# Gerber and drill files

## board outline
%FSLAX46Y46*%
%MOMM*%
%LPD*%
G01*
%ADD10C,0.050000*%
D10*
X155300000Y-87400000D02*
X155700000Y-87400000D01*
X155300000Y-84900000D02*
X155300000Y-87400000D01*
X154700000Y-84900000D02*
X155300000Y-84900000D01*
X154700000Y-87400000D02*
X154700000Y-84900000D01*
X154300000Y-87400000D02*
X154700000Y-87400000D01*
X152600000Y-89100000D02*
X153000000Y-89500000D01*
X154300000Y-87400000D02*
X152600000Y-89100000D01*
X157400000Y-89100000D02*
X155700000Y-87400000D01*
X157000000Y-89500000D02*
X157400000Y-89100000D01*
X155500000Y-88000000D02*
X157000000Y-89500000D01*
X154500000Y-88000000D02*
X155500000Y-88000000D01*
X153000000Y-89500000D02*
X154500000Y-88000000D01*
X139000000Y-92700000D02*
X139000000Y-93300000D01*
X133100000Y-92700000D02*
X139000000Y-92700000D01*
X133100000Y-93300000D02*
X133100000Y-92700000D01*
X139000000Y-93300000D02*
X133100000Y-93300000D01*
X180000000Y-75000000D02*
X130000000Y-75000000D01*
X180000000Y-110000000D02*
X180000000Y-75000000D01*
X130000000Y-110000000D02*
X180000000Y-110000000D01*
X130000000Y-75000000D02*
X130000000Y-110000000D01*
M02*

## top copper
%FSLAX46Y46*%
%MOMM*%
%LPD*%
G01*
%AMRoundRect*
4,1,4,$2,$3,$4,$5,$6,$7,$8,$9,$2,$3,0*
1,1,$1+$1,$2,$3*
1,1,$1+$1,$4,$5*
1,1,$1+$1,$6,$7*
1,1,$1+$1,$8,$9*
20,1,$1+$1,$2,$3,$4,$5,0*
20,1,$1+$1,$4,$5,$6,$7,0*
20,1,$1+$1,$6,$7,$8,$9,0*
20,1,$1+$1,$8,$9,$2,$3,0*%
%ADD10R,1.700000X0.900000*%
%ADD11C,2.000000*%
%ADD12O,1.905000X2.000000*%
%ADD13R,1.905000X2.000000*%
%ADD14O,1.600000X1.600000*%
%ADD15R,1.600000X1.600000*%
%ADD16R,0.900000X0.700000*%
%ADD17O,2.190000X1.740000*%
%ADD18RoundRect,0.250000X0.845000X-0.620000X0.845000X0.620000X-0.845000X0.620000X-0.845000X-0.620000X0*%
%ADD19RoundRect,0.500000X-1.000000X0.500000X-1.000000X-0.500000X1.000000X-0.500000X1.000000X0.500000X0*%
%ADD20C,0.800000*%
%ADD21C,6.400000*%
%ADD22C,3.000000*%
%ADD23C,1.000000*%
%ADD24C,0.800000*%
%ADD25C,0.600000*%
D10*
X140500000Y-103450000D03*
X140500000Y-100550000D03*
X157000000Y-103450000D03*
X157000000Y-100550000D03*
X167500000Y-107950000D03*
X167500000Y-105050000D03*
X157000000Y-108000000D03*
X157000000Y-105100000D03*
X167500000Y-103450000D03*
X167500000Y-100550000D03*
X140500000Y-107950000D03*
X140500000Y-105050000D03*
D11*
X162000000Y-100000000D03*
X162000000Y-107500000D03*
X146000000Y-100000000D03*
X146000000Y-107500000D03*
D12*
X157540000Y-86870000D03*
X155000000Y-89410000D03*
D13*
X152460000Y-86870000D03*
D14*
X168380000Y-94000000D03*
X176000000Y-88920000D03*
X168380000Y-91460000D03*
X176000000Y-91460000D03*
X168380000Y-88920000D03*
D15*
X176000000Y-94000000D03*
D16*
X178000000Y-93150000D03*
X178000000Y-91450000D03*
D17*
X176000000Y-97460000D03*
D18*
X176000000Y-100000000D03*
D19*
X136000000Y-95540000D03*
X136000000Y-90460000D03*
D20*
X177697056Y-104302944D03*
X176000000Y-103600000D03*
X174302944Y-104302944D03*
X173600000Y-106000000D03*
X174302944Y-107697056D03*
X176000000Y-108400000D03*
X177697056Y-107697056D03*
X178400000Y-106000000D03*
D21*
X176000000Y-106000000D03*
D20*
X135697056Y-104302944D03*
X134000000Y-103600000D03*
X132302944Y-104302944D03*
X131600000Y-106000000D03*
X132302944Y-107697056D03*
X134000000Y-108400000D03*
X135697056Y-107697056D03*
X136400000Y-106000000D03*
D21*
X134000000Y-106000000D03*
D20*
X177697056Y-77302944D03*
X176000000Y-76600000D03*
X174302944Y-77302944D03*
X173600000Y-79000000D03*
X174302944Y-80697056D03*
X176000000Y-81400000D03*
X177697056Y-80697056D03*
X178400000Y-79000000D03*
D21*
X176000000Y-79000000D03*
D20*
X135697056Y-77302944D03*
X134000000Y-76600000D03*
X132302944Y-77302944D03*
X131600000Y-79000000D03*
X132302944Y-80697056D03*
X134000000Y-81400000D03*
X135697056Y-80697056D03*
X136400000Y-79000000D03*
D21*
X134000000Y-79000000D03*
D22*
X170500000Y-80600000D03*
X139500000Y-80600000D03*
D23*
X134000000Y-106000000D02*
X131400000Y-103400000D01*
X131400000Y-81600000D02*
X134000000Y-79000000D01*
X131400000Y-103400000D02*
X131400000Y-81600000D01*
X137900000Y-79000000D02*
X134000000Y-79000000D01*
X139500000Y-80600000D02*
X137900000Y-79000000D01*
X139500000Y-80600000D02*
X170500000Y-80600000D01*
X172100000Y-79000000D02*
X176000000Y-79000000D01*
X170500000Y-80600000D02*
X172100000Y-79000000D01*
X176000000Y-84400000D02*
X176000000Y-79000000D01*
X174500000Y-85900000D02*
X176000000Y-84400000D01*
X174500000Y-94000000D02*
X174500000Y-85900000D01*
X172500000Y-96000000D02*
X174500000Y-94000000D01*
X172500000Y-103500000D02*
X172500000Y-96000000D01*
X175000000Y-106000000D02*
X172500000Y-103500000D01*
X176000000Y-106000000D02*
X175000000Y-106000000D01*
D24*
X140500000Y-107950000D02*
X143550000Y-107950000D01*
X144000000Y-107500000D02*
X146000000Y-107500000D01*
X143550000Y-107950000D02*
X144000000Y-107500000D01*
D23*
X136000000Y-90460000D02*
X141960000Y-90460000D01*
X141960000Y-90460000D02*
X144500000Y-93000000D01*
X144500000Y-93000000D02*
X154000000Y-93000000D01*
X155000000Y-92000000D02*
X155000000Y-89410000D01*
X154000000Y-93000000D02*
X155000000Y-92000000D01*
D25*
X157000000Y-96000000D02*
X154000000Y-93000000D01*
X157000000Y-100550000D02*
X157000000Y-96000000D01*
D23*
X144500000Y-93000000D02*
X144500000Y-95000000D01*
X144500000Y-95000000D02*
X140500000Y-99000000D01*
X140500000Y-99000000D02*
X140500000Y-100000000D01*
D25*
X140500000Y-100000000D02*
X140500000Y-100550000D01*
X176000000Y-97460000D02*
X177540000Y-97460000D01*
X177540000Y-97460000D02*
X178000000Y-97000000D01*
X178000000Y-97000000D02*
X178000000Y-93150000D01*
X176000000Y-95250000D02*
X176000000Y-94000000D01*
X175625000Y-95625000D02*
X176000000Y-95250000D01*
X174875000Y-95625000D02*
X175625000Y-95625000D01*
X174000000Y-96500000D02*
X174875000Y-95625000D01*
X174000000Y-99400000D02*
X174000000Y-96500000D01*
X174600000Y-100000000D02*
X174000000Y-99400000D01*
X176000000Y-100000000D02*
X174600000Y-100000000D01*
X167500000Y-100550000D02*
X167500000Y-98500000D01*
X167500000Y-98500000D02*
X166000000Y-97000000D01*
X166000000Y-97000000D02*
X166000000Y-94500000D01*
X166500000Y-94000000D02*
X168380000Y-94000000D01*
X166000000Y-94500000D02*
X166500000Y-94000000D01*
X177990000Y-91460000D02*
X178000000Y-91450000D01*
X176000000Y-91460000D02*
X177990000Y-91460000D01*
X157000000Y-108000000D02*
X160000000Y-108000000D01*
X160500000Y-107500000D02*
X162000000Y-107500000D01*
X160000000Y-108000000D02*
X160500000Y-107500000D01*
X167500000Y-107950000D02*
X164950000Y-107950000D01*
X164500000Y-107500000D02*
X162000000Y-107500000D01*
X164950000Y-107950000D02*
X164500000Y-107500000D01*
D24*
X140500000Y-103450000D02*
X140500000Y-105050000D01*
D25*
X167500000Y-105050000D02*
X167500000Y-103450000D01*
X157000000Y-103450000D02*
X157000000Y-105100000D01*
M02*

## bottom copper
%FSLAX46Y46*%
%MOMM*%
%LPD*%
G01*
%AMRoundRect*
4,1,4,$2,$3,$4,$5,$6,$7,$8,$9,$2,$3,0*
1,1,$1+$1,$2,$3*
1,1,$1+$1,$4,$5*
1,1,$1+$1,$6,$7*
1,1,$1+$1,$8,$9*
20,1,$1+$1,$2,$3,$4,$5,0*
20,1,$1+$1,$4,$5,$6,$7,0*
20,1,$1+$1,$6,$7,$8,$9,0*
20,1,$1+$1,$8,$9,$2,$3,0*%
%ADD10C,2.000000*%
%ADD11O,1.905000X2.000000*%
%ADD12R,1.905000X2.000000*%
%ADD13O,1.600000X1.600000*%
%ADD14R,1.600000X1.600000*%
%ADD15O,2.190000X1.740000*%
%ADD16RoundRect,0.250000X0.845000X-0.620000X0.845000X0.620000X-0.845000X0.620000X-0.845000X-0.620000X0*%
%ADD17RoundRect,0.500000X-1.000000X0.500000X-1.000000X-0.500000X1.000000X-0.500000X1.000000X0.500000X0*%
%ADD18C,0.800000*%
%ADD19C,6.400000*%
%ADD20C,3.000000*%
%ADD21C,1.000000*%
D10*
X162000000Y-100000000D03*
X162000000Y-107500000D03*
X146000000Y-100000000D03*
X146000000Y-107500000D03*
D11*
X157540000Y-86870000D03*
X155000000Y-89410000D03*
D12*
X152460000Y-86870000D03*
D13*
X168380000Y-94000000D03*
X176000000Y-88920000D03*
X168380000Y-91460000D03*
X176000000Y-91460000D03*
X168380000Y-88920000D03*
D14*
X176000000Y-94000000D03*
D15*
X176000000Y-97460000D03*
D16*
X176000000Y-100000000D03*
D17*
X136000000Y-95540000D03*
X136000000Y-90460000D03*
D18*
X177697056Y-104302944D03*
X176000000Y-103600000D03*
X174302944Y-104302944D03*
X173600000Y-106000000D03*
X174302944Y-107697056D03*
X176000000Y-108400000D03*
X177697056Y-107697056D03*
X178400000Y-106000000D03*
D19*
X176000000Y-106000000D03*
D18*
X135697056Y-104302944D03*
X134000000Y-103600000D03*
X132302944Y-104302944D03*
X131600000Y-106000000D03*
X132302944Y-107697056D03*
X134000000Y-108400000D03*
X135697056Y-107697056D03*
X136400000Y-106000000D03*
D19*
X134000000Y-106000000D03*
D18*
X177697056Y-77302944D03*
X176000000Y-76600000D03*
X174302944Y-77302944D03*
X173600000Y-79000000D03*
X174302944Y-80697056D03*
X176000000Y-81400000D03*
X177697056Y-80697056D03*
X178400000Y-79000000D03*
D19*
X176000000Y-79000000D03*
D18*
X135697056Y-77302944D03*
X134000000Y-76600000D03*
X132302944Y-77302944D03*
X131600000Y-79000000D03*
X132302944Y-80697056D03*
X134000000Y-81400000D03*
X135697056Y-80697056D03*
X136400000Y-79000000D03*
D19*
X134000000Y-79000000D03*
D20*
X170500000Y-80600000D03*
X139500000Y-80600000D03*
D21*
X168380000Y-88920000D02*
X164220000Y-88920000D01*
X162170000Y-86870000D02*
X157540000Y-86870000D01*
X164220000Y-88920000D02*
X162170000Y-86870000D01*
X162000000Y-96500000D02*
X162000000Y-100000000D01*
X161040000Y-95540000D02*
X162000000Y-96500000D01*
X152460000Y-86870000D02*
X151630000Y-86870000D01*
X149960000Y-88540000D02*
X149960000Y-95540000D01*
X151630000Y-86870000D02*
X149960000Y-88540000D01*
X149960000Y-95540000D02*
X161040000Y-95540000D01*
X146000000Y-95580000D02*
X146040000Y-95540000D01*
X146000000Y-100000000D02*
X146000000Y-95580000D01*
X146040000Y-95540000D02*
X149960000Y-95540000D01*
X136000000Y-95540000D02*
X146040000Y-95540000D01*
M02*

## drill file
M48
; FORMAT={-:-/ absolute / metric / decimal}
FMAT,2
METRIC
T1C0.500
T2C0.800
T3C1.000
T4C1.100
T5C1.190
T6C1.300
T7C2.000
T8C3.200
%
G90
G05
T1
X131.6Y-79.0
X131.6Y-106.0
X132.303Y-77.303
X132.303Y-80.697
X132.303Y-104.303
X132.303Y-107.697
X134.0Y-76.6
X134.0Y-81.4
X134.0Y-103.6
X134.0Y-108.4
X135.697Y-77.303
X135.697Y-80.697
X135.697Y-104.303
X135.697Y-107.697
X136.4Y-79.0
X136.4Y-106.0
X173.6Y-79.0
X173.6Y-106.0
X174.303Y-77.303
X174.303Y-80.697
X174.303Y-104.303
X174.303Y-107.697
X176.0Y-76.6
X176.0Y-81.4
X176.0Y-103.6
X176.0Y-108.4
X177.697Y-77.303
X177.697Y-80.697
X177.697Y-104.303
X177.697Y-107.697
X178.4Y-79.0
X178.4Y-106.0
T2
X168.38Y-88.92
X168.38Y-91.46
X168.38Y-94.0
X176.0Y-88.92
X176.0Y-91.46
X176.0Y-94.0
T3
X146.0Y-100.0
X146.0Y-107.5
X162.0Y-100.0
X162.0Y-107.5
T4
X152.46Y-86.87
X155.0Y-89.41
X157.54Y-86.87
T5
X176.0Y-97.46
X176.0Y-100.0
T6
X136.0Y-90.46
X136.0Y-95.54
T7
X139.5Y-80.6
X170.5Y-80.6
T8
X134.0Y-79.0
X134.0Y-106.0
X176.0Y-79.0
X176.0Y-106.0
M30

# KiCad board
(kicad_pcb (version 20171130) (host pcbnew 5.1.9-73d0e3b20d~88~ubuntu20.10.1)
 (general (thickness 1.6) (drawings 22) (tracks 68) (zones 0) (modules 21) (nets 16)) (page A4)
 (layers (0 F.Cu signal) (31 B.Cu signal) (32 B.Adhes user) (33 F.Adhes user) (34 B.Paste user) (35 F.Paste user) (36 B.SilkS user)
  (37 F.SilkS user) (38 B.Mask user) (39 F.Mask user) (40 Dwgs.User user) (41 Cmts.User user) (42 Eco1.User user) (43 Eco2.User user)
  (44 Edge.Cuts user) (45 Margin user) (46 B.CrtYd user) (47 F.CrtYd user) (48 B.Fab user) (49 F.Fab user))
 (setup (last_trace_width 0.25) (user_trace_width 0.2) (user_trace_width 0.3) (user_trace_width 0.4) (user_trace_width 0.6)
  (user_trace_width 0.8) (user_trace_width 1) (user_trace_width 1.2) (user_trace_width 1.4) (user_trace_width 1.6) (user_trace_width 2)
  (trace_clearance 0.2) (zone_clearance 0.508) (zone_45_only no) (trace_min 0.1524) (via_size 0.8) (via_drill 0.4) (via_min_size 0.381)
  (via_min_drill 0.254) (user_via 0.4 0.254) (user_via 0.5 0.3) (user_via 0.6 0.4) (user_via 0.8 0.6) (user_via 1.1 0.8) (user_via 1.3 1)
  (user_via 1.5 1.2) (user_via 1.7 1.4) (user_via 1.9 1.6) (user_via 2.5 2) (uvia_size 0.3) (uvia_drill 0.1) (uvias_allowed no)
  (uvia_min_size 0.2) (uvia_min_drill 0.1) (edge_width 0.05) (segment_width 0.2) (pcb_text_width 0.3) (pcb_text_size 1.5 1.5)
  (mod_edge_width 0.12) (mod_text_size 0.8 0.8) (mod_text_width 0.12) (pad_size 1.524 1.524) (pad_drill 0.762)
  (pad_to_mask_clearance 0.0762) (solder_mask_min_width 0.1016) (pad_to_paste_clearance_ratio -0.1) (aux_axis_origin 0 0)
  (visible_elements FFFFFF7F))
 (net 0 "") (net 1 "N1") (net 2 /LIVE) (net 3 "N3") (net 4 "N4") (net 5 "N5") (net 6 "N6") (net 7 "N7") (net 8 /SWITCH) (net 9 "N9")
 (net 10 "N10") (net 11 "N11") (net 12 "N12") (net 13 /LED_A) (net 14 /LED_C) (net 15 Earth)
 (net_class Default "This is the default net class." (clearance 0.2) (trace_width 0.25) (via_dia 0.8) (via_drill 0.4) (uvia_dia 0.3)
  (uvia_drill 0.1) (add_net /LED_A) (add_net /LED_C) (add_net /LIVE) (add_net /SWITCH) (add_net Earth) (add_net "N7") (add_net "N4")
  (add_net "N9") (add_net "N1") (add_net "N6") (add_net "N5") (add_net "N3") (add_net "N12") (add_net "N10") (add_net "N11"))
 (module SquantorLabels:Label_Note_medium (layer F.Cu) (at 156.5 94.2)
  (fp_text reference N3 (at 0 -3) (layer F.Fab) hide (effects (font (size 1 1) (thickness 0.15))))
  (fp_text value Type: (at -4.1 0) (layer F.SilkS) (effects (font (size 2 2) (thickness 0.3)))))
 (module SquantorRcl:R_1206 (layer F.Cu) (at 140.5 102 270)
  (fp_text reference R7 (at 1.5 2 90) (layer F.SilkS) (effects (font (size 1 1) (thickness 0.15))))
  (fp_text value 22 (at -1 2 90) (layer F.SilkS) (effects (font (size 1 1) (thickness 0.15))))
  (pad 2 smd rect (at 1.45 0 270) (size 0.9 1.7) (layers F.Cu F.Paste F.Mask) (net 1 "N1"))
  (pad 1 smd rect (at -1.45 0 270) (size 0.9 1.7) (layers F.Cu F.Paste F.Mask) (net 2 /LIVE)))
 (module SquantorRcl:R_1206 (layer F.Cu) (at 157 102 270)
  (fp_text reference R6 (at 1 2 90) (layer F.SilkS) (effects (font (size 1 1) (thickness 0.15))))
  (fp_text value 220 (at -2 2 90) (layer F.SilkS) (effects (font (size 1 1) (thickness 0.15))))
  (pad 2 smd rect (at 1.45 0 270) (size 0.9 1.7) (layers F.Cu F.Paste F.Mask) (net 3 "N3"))
  (pad 1 smd rect (at -1.45 0 270) (size 0.9 1.7) (layers F.Cu F.Paste F.Mask) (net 2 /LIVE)))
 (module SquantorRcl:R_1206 (layer F.Cu) (at 167.5 106.5 270)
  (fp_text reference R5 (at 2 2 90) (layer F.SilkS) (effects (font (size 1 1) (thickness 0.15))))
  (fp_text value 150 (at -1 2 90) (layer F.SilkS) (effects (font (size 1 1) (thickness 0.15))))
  (pad 2 smd rect (at 1.45 0 270) (size 0.9 1.7) (layers F.Cu F.Paste F.Mask) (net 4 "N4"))
  (pad 1 smd rect (at -1.45 0 270) (size 0.9 1.7) (layers F.Cu F.Paste F.Mask) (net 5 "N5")))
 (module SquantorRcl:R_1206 (layer F.Cu) (at 157 106.55 270)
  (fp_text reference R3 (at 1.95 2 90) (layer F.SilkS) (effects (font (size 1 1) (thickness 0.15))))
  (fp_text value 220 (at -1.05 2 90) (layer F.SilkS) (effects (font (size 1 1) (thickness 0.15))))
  (pad 2 smd rect (at 1.45 0 270) (size 0.9 1.7) (layers F.Cu F.Paste F.Mask) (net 4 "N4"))
  (pad 1 smd rect (at -1.45 0 270) (size 0.9 1.7) (layers F.Cu F.Paste F.Mask) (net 3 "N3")))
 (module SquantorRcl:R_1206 (layer F.Cu) (at 167.5 102 270)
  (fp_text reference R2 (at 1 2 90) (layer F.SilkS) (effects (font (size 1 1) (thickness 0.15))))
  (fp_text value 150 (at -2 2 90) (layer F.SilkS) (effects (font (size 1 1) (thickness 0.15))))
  (pad 2 smd rect (at 1.45 0 270) (size 0.9 1.7) (layers F.Cu F.Paste F.Mask) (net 5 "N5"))
  (pad 1 smd rect (at -1.45 0 270) (size 0.9 1.7) (layers F.Cu F.Paste F.Mask) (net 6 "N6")))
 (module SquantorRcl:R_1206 (layer F.Cu) (at 140.5 106.5 270)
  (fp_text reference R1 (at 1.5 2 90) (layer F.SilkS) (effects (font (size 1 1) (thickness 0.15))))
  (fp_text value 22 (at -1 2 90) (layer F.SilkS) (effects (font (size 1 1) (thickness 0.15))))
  (pad 2 smd rect (at 1.45 0 270) (size 0.9 1.7) (layers F.Cu F.Paste F.Mask) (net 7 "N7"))
  (pad 1 smd rect (at -1.45 0 270) (size 0.9 1.7) (layers F.Cu F.Paste F.Mask) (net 1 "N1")))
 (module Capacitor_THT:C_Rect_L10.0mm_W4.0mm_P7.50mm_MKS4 (layer F.Cu) (at 162 107.5 90)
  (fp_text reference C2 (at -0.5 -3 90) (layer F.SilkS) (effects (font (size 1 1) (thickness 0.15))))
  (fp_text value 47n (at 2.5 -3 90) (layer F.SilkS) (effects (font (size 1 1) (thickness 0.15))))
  (pad 2 thru_hole circle (at 7.5 0 90) (size 2 2) (drill 1) (layers *.Cu *.Mask) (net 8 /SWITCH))
  (pad 1 thru_hole circle (at 0 0 90) (size 2 2) (drill 1) (layers *.Cu *.Mask) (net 4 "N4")))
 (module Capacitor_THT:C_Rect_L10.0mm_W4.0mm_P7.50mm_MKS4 (layer F.Cu) (at 146 107.5 90)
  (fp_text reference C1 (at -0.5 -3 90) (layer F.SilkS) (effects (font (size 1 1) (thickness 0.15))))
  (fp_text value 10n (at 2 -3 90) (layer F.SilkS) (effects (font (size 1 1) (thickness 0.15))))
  (pad 2 thru_hole circle (at 7.5 0 90) (size 2 2) (drill 1) (layers *.Cu *.Mask) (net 8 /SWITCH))
  (pad 1 thru_hole circle (at 0 0 90) (size 2 2) (drill 1) (layers *.Cu *.Mask) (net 7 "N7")))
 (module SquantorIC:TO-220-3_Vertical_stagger (layer F.Cu) (at 155 85.6)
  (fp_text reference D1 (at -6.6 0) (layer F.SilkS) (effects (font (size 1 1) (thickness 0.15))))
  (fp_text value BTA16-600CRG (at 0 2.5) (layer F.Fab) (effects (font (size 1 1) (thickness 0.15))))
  (pad 3 thru_hole oval (at 2.54 1.27) (size 1.905 2) (drill 1.1) (layers *.Cu *.Mask) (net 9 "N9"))
  (pad 2 thru_hole oval (at 0 3.81) (size 1.905 2) (drill 1.1) (layers *.Cu *.Mask) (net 2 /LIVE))
  (pad 1 thru_hole rect (at -2.54 1.27) (size 1.905 2) (drill 1.1) (layers *.Cu *.Mask) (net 8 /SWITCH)))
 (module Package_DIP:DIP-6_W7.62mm (layer F.Cu) (at 176 94 180)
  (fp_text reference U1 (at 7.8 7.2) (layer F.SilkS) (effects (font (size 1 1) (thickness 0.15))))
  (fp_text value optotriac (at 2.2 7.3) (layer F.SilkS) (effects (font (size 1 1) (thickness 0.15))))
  (pad 6 thru_hole oval (at 7.62 0 180) (size 1.6 1.6) (drill 0.8) (layers *.Cu *.Mask) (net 6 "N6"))
  (pad 3 thru_hole oval (at 0 5.08 180) (size 1.6 1.6) (drill 0.8) (layers *.Cu *.Mask) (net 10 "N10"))
  (pad 5 thru_hole oval (at 7.62 2.54 180) (size 1.6 1.6) (drill 0.8) (layers *.Cu *.Mask) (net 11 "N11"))
  (pad 2 thru_hole oval (at 0 2.54 180) (size 1.6 1.6) (drill 0.8) (layers *.Cu *.Mask) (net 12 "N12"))
  (pad 4 thru_hole oval (at 7.62 5.08 180) (size 1.6 1.6) (drill 0.8) (layers *.Cu *.Mask) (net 9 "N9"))
  (pad 1 thru_hole rect (at 0 0 180) (size 1.6 1.6) (drill 0.8) (layers *.Cu *.Mask) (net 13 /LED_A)))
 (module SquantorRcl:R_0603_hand (layer F.Cu) (at 178 92.3 270)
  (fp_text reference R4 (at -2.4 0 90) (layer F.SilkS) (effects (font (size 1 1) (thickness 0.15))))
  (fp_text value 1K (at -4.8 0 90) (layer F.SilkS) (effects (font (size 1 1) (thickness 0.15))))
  (pad 2 smd rect (at 0.85 0 270) (size 0.7 0.9) (layers F.Cu F.Paste F.Mask) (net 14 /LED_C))
  (pad 1 smd rect (at -0.85 0 270) (size 0.7 0.9) (layers F.Cu F.Paste F.Mask) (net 12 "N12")))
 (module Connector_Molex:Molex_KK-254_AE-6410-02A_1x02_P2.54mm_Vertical (layer F.Cu) (at 176 100 90)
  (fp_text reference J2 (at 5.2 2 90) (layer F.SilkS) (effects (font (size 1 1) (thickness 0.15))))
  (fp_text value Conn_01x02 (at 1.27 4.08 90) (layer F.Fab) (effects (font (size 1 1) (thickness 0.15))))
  (pad 2 thru_hole oval (at 2.54 0 90) (size 1.74 2.19) (drill 1.19) (layers *.Cu *.Mask) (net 14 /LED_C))
  (pad 1 thru_hole roundrect (at 0 0 90) (size 1.74 2.19) (drill 1.19) (layers *.Cu *.Mask) (roundrect_rratio 0.143678) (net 13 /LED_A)))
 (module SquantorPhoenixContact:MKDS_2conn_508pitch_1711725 (layer F.Cu) (at 136 93 270)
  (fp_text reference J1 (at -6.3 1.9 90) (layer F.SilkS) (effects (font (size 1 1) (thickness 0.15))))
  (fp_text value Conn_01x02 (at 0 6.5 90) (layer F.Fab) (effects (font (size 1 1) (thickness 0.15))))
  (pad 2 thru_hole roundrect (at 2.54 0 270) (size 2 3) (drill 1.3) (layers *.Cu *.Mask) (roundrect_rratio 0.25) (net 8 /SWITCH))
  (pad 1 thru_hole roundrect (at -2.54 0 270) (size 2 3) (drill 1.3) (layers *.Cu *.Mask) (roundrect_rratio 0.25) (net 2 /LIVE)))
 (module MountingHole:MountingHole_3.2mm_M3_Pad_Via (layer F.Cu) (at 176 106)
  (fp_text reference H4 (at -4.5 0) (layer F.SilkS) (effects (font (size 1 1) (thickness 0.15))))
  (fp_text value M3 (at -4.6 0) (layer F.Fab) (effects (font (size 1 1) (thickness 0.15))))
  (pad 1 thru_hole circle (at 1.697056 -1.697056) (size 0.8 0.8) (drill 0.5) (layers *.Cu *.Mask) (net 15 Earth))
  (pad 1 thru_hole circle (at 0 -2.4) (size 0.8 0.8) (drill 0.5) (layers *.Cu *.Mask) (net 15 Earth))
  (pad 1 thru_hole circle (at -1.697056 -1.697056) (size 0.8 0.8) (drill 0.5) (layers *.Cu *.Mask) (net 15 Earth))
  (pad 1 thru_hole circle (at -2.4 0) (size 0.8 0.8) (drill 0.5) (layers *.Cu *.Mask) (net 15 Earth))
  (pad 1 thru_hole circle (at -1.697056 1.697056) (size 0.8 0.8) (drill 0.5) (layers *.Cu *.Mask) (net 15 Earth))
  (pad 1 thru_hole circle (at 0 2.4) (size 0.8 0.8) (drill 0.5) (layers *.Cu *.Mask) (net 15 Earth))
  (pad 1 thru_hole circle (at 1.697056 1.697056) (size 0.8 0.8) (drill 0.5) (layers *.Cu *.Mask) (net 15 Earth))
  (pad 1 thru_hole circle (at 2.4 0) (size 0.8 0.8) (drill 0.5) (layers *.Cu *.Mask) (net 15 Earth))
  (pad 1 thru_hole circle (at 0 0) (size 6.4 6.4) (drill 3.2) (layers *.Cu *.Mask) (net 15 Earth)))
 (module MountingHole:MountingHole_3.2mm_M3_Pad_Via (layer F.Cu) (at 134 106)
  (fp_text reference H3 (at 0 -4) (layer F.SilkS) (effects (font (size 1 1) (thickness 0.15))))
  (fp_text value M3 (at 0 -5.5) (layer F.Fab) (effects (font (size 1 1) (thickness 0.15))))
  (pad 1 thru_hole circle (at 1.697056 -1.697056) (size 0.8 0.8) (drill 0.5) (layers *.Cu *.Mask) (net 15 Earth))
  (pad 1 thru_hole circle (at 0 -2.4) (size 0.8 0.8) (drill 0.5) (layers *.Cu *.Mask) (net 15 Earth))
  (pad 1 thru_hole circle (at -1.697056 -1.697056) (size 0.8 0.8) (drill 0.5) (layers *.Cu *.Mask) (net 15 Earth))
  (pad 1 thru_hole circle (at -2.4 0) (size 0.8 0.8) (drill 0.5) (layers *.Cu *.Mask) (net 15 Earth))
  (pad 1 thru_hole circle (at -1.697056 1.697056) (size 0.8 0.8) (drill 0.5) (layers *.Cu *.Mask) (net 15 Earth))
  (pad 1 thru_hole circle (at 0 2.4) (size 0.8 0.8) (drill 0.5) (layers *.Cu *.Mask) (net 15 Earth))
  (pad 1 thru_hole circle (at 1.697056 1.697056) (size 0.8 0.8) (drill 0.5) (layers *.Cu *.Mask) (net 15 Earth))
  (pad 1 thru_hole circle (at 2.4 0) (size 0.8 0.8) (drill 0.5) (layers *.Cu *.Mask) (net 15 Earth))
  (pad 1 thru_hole circle (at 0 0) (size 6.4 6.4) (drill 3.2) (layers *.Cu *.Mask) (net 15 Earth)))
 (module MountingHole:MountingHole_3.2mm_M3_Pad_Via (layer F.Cu) (at 176 79)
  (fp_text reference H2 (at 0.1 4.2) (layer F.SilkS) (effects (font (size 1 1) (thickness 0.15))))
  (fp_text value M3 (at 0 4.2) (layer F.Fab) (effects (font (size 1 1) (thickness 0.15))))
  (pad 1 thru_hole circle (at 1.697056 -1.697056) (size 0.8 0.8) (drill 0.5) (layers *.Cu *.Mask) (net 15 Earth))
  (pad 1 thru_hole circle (at 0 -2.4) (size 0.8 0.8) (drill 0.5) (layers *.Cu *.Mask) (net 15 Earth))
  (pad 1 thru_hole circle (at -1.697056 -1.697056) (size 0.8 0.8) (drill 0.5) (layers *.Cu *.Mask) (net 15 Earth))
  (pad 1 thru_hole circle (at -2.4 0) (size 0.8 0.8) (drill 0.5) (layers *.Cu *.Mask) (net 15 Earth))
  (pad 1 thru_hole circle (at -1.697056 1.697056) (size 0.8 0.8) (drill 0.5) (layers *.Cu *.Mask) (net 15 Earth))
  (pad 1 thru_hole circle (at 0 2.4) (size 0.8 0.8) (drill 0.5) (layers *.Cu *.Mask) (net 15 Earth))
  (pad 1 thru_hole circle (at 1.697056 1.697056) (size 0.8 0.8) (drill 0.5) (layers *.Cu *.Mask) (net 15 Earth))
  (pad 1 thru_hole circle (at 2.4 0) (size 0.8 0.8) (drill 0.5) (layers *.Cu *.Mask) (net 15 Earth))
  (pad 1 thru_hole circle (at 0 0) (size 6.4 6.4) (drill 3.2) (layers *.Cu *.Mask) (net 15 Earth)))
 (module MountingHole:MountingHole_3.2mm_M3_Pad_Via (layer F.Cu) (at 134 79)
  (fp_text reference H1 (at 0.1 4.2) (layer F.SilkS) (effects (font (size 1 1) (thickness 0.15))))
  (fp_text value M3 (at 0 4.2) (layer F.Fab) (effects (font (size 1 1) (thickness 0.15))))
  (pad 1 thru_hole circle (at 1.697056 -1.697056) (size 0.8 0.8) (drill 0.5) (layers *.Cu *.Mask) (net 15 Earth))
  (pad 1 thru_hole circle (at 0 -2.4) (size 0.8 0.8) (drill 0.5) (layers *.Cu *.Mask) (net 15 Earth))
  (pad 1 thru_hole circle (at -1.697056 -1.697056) (size 0.8 0.8) (drill 0.5) (layers *.Cu *.Mask) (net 15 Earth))
  (pad 1 thru_hole circle (at -2.4 0) (size 0.8 0.8) (drill 0.5) (layers *.Cu *.Mask) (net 15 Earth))
  (pad 1 thru_hole circle (at -1.697056 1.697056) (size 0.8 0.8) (drill 0.5) (layers *.Cu *.Mask) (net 15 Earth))
  (pad 1 thru_hole circle (at 0 2.4) (size 0.8 0.8) (drill 0.5) (layers *.Cu *.Mask) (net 15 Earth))
  (pad 1 thru_hole circle (at 1.697056 1.697056) (size 0.8 0.8) (drill 0.5) (layers *.Cu *.Mask) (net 15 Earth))
  (pad 1 thru_hole circle (at 2.4 0) (size 0.8 0.8) (drill 0.5) (layers *.Cu *.Mask) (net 15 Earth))
  (pad 1 thru_hole circle (at 0 0) (size 6.4 6.4) (drill 3.2) (layers *.Cu *.Mask) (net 15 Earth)))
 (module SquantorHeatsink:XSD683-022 (layer F.Cu) (at 155 80.6)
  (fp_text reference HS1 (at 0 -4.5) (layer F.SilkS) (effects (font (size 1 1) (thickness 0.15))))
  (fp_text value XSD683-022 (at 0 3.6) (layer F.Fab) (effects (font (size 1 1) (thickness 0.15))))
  (pad 2 thru_hole circle (at 15.5 0) (size 3 3) (drill 2) (layers *.Cu *.Mask) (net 15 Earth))
  (pad 1 thru_hole circle (at -15.5 0) (size 3 3) (drill 2) (layers *.Cu *.Mask) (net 15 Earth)))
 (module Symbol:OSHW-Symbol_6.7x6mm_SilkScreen (layer B.Cu) (at 155.2 80.2 180)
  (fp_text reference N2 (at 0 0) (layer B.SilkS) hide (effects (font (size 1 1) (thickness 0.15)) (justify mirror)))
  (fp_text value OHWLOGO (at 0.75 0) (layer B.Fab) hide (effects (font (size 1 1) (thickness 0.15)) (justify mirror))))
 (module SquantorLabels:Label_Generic (layer B.Cu) (at 155.8 84.1 180)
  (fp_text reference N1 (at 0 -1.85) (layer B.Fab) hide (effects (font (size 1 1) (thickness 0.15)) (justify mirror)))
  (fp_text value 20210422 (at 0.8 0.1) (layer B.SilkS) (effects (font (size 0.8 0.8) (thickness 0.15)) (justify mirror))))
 (gr_line (start 155.3 87.4) (end 155.7 87.4) (layer Edge.Cuts) (width 0.05))
 (gr_line (start 155.3 84.9) (end 155.3 87.4) (layer Edge.Cuts) (width 0.05))
 (gr_line (start 154.7 84.9) (end 155.3 84.9) (layer Edge.Cuts) (width 0.05))
 (gr_line (start 154.7 87.4) (end 154.7 84.9) (layer Edge.Cuts) (width 0.05))
 (gr_line (start 154.3 87.4) (end 154.7 87.4) (layer Edge.Cuts) (width 0.05))
 (gr_line (start 152.6 89.1) (end 153 89.5) (layer Edge.Cuts) (width 0.05))
 (gr_line (start 154.3 87.4) (end 152.6 89.1) (layer Edge.Cuts) (width 0.05))
 (gr_line (start 157.4 89.1) (end 155.7 87.4) (layer Edge.Cuts) (width 0.05))
 (gr_line (start 157 89.5) (end 157.4 89.1) (layer Edge.Cuts) (width 0.05))
 (gr_line (start 155.5 88) (end 157 89.5) (layer Edge.Cuts) (width 0.05))
 (gr_line (start 154.5 88) (end 155.5 88) (layer Edge.Cuts) (width 0.05))
 (gr_line (start 153 89.5) (end 154.5 88) (layer Edge.Cuts) (width 0.05))
 (gr_line (start 139 92.7) (end 139 93.3) (layer Edge.Cuts) (width 0.05))
 (gr_line (start 133.1 92.7) (end 139 92.7) (layer Edge.Cuts) (width 0.05))
 (gr_line (start 133.1 93.3) (end 133.1 92.7) (layer Edge.Cuts) (width 0.05))
 (gr_line (start 139 93.3) (end 133.1 93.3) (layer Edge.Cuts) (width 0.05))
 (gr_line (start 180 75) (end 130 75) (layer Edge.Cuts) (width 0.05))
 (gr_line (start 180 110) (end 180 75) (layer Edge.Cuts) (width 0.05))
 (gr_line (start 130 110) (end 180 110) (layer Edge.Cuts) (width 0.05))
 (gr_line (start 130 75) (end 130 110) (layer Edge.Cuts) (width 0.05))
 (segment (start 168.38 88.92) (end 164.22 88.92) (width 1) (layer B.Cu) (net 9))
 (segment (start 162.17 86.87) (end 157.54 86.87) (width 1) (layer B.Cu) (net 9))
 (segment (start 164.22 88.92) (end 162.17 86.87) (width 1) (layer B.Cu) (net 9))
 (segment (start 134 106) (end 131.4 103.4) (width 1) (layer F.Cu) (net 15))
 (segment (start 131.4 81.6) (end 134 79) (width 1) (layer F.Cu) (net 15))
 (segment (start 131.4 103.4) (end 131.4 81.6) (width 1) (layer F.Cu) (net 15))
 (segment (start 137.9 79) (end 134 79) (width 1) (layer F.Cu) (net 15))
 (segment (start 139.5 80.6) (end 137.9 79) (width 1) (layer F.Cu) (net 15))
 (segment (start 139.5 80.6) (end 170.5 80.6) (width 1) (layer F.Cu) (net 15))
 (segment (start 172.1 79) (end 176 79) (width 1) (layer F.Cu) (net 15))
 (segment (start 170.5 80.6) (end 172.1 79) (width 1) (layer F.Cu) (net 15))
 (segment (start 176 84.4) (end 176 79) (width 1) (layer F.Cu) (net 15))
 (segment (start 174.5 85.9) (end 176 84.4) (width 1) (layer F.Cu) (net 15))
 (segment (start 174.5 94) (end 174.5 85.9) (width 1) (layer F.Cu) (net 15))
 (segment (start 172.5 96) (end 174.5 94) (width 1) (layer F.Cu) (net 15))
 (segment (start 172.5 103.5) (end 172.5 96) (width 1) (layer F.Cu) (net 15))
 (segment (start 175 106) (end 172.5 103.5) (width 1) (layer F.Cu) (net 15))
 (segment (start 176 106) (end 175 106) (width 1) (layer F.Cu) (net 15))
 (segment (start 140.5 107.95) (end 143.55 107.95) (width 0.8) (layer F.Cu) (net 7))
 (segment (start 144 107.5) (end 146 107.5) (width 0.8) (layer F.Cu) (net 7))
 (segment (start 143.55 107.95) (end 144 107.5) (width 0.8) (layer F.Cu) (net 7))
 (segment (start 136 90.46) (end 141.96 90.46) (width 1) (layer F.Cu) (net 2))
 (segment (start 141.96 90.46) (end 144.5 93) (width 1) (layer F.Cu) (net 2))
 (segment (start 144.5 93) (end 154 93) (width 1) (layer F.Cu) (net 2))
 (segment (start 155 92) (end 155 89.41) (width 1) (layer F.Cu) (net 2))
 (segment (start 154 93) (end 155 92) (width 1) (layer F.Cu) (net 2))
 (segment (start 157 96) (end 154 93) (width 0.6) (layer F.Cu) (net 2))
 (segment (start 157 100.55) (end 157 96) (width 0.6) (layer F.Cu) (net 2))
 (segment (start 144.5 93) (end 144.5 95) (width 1) (layer F.Cu) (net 2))
 (segment (start 144.5 95) (end 140.5 99) (width 1) (layer F.Cu) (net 2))
 (segment (start 140.5 99) (end 140.5 100) (width 1) (layer F.Cu) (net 2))
 (segment (start 140.5 100) (end 140.5 100.55) (width 0.6) (layer F.Cu) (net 2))
 (segment (start 162 96.5) (end 162 100) (width 1) (layer B.Cu) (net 8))
 (segment (start 161.04 95.54) (end 162 96.5) (width 1) (layer B.Cu) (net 8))
 (segment (start 152.46 86.87) (end 151.63 86.87) (width 1) (layer B.Cu) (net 8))
 (segment (start 149.96 88.54) (end 149.96 95.54) (width 1) (layer B.Cu) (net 8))
 (segment (start 151.63 86.87) (end 149.96 88.54) (width 1) (layer B.Cu) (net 8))
 (segment (start 149.96 95.54) (end 161.04 95.54) (width 1) (layer B.Cu) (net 8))
 (segment (start 146 95.58) (end 146.04 95.54) (width 1) (layer B.Cu) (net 8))
 (segment (start 146 100) (end 146 95.58) (width 1) (layer B.Cu) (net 8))
 (segment (start 146.04 95.54) (end 149.96 95.54) (width 1) (layer B.Cu) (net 8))
 (segment (start 136 95.54) (end 146.04 95.54) (width 1) (layer B.Cu) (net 8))
 (segment (start 176 97.46) (end 177.54 97.46) (width 0.6) (layer F.Cu) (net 14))
 (segment (start 177.54 97.46) (end 178 97) (width 0.6) (layer F.Cu) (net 14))
 (segment (start 178 97) (end 178 93.15) (width 0.6) (layer F.Cu) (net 14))
 (segment (start 176 95.25) (end 176 94) (width 0.6) (layer F.Cu) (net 13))
 (segment (start 175.625 95.625) (end 176 95.25) (width 0.6) (layer F.Cu) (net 13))
 (segment (start 174.875 95.625) (end 175.625 95.625) (width 0.6) (layer F.Cu) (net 13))
 (segment (start 174 96.5) (end 174.875 95.625) (width 0.6) (layer F.Cu) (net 13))
 (segment (start 174 99.4) (end 174 96.5) (width 0.6) (layer F.Cu) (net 13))
 (segment (start 174.6 100) (end 174 99.4) (width 0.6) (layer F.Cu) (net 13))
 (segment (start 176 100) (end 174.6 100) (width 0.6) (layer F.Cu) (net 13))
 (segment (start 167.5 100.55) (end 167.5 98.5) (width 0.6) (layer F.Cu) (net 6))
 (segment (start 167.5 98.5) (end 166 97) (width 0.6) (layer F.Cu) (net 6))
 (segment (start 166 97) (end 166 94.5) (width 0.6) (layer F.Cu) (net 6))
 (segment (start 166.5 94) (end 168.38 94) (width 0.6) (layer F.Cu) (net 6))
 (segment (start 166 94.5) (end 166.5 94) (width 0.6) (layer F.Cu) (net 6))
 (segment (start 177.99 91.46) (end 178 91.45) (width 0.6) (layer F.Cu) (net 12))
 (segment (start 176 91.46) (end 177.99 91.46) (width 0.6) (layer F.Cu) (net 12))
 (segment (start 157 108) (end 160 108) (width 0.6) (layer F.Cu) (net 4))
 (segment (start 160.5 107.5) (end 162 107.5) (width 0.6) (layer F.Cu) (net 4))
 (segment (start 160 108) (end 160.5 107.5) (width 0.6) (layer F.Cu) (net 4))
 (segment (start 167.5 107.95) (end 164.95 107.95) (width 0.6) (layer F.Cu) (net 4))
 (segment (start 164.5 107.5) (end 162 107.5) (width 0.6) (layer F.Cu) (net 4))
 (segment (start 164.95 107.95) (end 164.5 107.5) (width 0.6) (layer F.Cu) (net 4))
 (segment (start 140.5 103.45) (end 140.5 105.05) (width 0.8) (layer F.Cu) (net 1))
 (segment (start 167.5 105.05) (end 167.5 103.45) (width 0.6) (layer F.Cu) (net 5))
 (segment (start 157 103.45) (end 157 105.1) (width 0.6) (layer F.Cu) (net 3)))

